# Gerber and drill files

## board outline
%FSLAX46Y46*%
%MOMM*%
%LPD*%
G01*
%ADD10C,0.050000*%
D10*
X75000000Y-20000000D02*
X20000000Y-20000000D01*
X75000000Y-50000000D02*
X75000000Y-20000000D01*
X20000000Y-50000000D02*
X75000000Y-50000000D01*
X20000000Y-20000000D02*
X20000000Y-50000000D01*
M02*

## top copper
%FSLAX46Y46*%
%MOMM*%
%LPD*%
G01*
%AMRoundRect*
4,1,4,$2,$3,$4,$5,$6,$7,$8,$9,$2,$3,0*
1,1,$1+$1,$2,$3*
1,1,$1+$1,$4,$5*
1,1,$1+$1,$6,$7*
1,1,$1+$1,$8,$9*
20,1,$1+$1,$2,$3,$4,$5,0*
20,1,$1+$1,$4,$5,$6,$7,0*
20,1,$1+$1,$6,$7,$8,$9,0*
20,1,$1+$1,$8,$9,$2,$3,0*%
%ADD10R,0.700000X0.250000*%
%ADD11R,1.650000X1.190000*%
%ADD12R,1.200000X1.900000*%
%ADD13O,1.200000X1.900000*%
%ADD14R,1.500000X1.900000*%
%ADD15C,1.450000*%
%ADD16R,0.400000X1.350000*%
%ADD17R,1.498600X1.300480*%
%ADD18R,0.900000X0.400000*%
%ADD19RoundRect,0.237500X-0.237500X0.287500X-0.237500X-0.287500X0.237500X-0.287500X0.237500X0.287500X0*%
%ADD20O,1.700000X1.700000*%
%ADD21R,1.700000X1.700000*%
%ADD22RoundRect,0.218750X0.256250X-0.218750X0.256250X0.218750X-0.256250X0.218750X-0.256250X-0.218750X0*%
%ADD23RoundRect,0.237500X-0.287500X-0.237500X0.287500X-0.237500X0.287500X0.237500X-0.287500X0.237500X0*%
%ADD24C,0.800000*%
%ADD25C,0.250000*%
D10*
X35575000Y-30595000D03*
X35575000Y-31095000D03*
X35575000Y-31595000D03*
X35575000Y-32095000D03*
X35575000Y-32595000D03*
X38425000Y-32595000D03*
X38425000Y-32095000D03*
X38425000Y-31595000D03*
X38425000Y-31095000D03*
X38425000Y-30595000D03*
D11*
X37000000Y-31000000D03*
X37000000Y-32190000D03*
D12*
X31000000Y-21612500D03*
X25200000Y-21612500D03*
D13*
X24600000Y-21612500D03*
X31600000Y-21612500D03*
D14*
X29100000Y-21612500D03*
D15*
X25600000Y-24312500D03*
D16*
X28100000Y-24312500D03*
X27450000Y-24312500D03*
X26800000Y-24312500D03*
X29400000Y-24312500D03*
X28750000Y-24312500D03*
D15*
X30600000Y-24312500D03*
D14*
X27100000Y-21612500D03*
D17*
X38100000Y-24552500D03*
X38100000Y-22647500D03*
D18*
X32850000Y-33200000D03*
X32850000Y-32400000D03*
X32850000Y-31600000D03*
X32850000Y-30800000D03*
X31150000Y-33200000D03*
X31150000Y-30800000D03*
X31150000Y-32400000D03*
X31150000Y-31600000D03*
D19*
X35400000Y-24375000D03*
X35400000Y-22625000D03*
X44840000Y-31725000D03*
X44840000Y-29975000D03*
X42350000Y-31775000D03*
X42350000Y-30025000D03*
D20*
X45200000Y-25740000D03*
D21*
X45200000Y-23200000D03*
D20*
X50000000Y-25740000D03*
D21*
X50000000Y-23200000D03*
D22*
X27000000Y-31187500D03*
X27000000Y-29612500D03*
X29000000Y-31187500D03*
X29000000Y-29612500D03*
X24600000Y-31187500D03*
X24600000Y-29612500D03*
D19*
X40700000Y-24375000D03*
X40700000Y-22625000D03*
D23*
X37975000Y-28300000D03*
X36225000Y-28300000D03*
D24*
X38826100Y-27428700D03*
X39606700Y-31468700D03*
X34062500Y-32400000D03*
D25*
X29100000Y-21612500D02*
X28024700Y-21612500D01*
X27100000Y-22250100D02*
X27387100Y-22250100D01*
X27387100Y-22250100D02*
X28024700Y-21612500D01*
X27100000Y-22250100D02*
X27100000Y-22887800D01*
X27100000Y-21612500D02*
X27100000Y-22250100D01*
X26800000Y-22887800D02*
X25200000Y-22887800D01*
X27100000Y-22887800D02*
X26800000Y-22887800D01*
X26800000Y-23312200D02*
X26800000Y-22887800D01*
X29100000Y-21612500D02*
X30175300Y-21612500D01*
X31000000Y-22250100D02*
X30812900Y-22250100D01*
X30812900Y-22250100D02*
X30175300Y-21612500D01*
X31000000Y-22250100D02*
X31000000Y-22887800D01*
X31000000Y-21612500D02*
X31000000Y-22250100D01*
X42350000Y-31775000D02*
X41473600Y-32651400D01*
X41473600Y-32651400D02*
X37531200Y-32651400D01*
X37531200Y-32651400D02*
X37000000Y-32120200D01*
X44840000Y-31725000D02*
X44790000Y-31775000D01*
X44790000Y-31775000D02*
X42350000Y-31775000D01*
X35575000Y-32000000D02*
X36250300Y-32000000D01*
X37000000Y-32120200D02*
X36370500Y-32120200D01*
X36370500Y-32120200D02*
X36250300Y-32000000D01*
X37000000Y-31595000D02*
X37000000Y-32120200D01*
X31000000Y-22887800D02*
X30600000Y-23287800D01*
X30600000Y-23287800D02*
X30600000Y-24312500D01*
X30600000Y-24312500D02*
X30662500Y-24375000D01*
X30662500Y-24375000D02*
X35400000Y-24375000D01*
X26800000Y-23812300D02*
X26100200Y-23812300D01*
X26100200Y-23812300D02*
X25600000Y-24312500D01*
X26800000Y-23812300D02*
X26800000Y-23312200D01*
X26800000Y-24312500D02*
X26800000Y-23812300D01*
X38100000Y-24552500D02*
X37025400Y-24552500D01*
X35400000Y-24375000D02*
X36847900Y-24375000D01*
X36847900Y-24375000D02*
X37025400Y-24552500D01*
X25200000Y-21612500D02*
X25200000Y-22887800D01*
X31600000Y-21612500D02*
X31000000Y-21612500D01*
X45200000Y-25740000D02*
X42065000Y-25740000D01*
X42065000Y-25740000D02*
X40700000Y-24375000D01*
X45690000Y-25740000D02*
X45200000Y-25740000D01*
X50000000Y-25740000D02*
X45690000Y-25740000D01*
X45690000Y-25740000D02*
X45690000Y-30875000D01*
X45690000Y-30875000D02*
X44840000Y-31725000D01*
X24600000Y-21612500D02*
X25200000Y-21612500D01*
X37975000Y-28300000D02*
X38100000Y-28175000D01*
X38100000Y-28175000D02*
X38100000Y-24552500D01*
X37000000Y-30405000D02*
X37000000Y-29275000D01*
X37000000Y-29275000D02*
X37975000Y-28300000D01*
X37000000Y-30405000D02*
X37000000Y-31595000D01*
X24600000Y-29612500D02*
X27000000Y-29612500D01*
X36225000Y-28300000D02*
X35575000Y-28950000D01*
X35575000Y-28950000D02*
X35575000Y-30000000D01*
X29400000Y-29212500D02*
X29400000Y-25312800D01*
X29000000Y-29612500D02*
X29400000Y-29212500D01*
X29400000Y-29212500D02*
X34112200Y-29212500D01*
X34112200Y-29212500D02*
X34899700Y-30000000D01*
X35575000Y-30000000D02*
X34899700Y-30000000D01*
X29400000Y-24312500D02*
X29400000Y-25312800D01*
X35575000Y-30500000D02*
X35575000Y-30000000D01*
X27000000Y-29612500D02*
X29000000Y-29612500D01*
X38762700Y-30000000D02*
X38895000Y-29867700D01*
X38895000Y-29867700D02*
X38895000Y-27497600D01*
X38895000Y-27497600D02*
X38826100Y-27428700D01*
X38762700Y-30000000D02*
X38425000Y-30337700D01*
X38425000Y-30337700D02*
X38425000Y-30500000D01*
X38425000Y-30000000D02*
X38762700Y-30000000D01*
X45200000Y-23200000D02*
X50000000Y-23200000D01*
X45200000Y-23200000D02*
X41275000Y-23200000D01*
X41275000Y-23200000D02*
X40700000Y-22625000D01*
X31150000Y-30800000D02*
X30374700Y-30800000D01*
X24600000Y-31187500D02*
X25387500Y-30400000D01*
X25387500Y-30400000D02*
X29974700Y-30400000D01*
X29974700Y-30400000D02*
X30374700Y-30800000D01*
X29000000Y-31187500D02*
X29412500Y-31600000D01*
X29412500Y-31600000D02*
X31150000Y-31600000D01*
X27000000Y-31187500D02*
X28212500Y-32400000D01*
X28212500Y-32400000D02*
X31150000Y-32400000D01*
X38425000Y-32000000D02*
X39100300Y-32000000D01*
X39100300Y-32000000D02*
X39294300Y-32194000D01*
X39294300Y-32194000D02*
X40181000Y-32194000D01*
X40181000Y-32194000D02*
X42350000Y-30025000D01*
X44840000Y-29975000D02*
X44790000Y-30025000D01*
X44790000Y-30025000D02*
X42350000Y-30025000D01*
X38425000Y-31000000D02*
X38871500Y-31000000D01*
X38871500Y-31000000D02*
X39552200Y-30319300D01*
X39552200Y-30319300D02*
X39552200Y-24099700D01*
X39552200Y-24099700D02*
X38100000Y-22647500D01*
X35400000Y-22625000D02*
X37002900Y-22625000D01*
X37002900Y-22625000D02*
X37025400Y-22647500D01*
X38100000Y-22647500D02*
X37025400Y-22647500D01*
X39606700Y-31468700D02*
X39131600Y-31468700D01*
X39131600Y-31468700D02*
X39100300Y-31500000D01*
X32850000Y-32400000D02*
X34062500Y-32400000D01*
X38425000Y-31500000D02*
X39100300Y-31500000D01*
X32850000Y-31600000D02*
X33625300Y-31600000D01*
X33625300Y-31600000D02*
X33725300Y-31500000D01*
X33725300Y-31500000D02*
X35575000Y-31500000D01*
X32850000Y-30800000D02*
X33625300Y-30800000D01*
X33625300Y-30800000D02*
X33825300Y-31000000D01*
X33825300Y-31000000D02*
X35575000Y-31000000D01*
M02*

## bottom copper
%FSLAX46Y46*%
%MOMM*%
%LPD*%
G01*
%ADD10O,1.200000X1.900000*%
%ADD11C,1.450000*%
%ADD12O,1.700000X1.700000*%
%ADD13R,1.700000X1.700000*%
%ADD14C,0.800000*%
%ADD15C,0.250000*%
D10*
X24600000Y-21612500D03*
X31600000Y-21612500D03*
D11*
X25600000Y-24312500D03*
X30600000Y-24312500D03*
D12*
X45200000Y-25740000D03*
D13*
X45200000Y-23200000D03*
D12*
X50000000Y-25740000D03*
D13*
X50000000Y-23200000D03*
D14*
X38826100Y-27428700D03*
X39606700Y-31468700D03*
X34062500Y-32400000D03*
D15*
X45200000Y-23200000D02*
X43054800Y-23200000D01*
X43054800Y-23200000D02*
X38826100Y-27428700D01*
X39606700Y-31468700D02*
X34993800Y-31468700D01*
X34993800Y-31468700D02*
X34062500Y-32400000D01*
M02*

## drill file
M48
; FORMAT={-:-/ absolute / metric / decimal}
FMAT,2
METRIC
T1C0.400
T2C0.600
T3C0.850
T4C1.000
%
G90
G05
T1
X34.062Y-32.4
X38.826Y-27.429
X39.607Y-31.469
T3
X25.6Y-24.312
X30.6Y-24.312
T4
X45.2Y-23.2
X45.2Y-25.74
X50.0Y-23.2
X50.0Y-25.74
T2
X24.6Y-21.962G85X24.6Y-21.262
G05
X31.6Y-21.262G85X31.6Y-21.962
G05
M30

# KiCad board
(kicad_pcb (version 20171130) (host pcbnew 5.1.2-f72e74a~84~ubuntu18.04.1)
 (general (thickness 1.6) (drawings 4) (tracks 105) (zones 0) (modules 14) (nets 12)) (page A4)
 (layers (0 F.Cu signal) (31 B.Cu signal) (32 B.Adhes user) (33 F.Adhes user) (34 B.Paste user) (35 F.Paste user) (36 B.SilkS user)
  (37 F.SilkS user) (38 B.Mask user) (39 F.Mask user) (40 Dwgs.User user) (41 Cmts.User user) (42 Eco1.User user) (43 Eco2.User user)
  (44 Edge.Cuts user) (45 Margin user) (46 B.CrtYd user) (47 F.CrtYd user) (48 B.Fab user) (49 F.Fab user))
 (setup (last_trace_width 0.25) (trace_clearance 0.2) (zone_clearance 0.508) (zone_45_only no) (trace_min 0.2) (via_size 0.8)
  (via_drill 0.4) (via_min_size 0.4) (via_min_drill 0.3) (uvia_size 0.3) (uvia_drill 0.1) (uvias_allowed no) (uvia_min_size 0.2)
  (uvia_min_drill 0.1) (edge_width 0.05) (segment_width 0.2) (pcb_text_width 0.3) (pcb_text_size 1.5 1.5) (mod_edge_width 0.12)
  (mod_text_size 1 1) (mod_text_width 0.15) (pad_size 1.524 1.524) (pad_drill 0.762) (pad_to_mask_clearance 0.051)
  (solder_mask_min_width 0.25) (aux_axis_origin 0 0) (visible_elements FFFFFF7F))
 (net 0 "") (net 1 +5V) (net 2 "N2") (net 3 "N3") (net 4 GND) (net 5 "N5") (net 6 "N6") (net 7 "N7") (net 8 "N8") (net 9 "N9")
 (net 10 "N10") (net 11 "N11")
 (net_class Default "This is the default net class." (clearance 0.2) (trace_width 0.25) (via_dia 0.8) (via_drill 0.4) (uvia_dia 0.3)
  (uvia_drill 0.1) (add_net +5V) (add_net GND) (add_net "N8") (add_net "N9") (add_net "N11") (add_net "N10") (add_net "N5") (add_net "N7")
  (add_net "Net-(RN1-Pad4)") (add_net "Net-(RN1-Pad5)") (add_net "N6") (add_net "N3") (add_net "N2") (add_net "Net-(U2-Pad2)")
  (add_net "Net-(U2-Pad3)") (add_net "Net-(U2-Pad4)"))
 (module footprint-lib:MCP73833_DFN (layer F.Cu) (at 37 31.595)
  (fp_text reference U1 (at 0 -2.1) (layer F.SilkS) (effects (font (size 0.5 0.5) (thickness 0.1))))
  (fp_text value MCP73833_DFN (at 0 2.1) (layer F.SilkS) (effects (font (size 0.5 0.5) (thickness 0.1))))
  (pad 1 smd rect (at -1.425 -1) (size 0.7 0.25) (layers F.Cu F.Paste F.Mask) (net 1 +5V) (solder_mask_margin 0.07))
  (pad 2 smd rect (at -1.425 -0.5) (size 0.7 0.25) (layers F.Cu F.Paste F.Mask) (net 1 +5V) (solder_mask_margin 0.07))
  (pad 3 smd rect (at -1.425 0) (size 0.7 0.25) (layers F.Cu F.Paste F.Mask) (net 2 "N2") (solder_mask_margin 0.07))
  (pad 4 smd rect (at -1.425 0.5) (size 0.7 0.25) (layers F.Cu F.Paste F.Mask) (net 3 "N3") (solder_mask_margin 0.07))
  (pad 5 smd rect (at -1.425 1) (size 0.7 0.25) (layers F.Cu F.Paste F.Mask) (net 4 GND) (solder_mask_margin 0.07))
  (pad 6 smd rect (at 1.425 1) (size 0.7 0.25) (layers F.Cu F.Paste F.Mask) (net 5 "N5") (solder_mask_margin 0.07))
  (pad 7 smd rect (at 1.425 0.5) (size 0.7 0.25) (layers F.Cu F.Paste F.Mask) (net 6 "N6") (solder_mask_margin 0.07))
  (pad 8 smd rect (at 1.425 0) (size 0.7 0.25) (layers F.Cu F.Paste F.Mask) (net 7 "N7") (solder_mask_margin 0.07))
  (pad 9 smd rect (at 1.425 -0.5) (size 0.7 0.25) (layers F.Cu F.Paste F.Mask) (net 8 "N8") (solder_mask_margin 0.07))
  (pad 10 smd rect (at 1.425 -1) (size 0.7 0.25) (layers F.Cu F.Paste F.Mask) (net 8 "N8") (solder_mask_margin 0.07))
  (pad 11 smd rect (at 0 -0.595) (size 1.65 1.19) (layers F.Cu F.Paste F.Mask) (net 4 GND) (solder_mask_margin 0.07)
   (solder_paste_margin -0.1))
  (pad 11 smd rect (at 0 0.595) (size 1.65 1.19) (layers F.Cu F.Paste F.Mask) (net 4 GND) (solder_mask_margin 0.07)
   (solder_paste_margin -0.1)))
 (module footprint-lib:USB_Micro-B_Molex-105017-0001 (layer F.Cu) (at 28.1 22.85 180)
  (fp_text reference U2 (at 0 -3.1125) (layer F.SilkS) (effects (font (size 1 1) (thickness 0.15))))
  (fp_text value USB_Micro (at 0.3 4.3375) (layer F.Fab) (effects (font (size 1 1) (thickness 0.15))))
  (pad 6 smd rect (at -2.9 1.2375 180) (size 1.2 1.9) (layers F.Cu F.Mask) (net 4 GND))
  (pad 7 smd rect (at 2.9 1.2375 180) (size 1.2 1.9) (layers F.Cu F.Mask) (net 4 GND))
  (pad 7 thru_hole oval (at 3.5 1.2375 180) (size 1.2 1.9) (drill oval 0.6 1.3) (layers *.Cu *.Mask) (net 4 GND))
  (pad 6 thru_hole oval (at -3.5 1.2375) (size 1.2 1.9) (drill oval 0.6 1.3) (layers *.Cu *.Mask) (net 4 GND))
  (pad 6 smd rect (at -1 1.2375 180) (size 1.5 1.9) (layers F.Cu F.Paste F.Mask) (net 4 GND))
  (pad 9 thru_hole circle (at 2.5 -1.4625 180) (size 1.45 1.45) (drill 0.85) (layers *.Cu *.Mask) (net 4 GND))
  (pad 3 smd rect (at 0 -1.4625 180) (size 0.4 1.35) (layers F.Cu F.Paste F.Mask))
  (pad 4 smd rect (at 0.65 -1.4625 180) (size 0.4 1.35) (layers F.Cu F.Paste F.Mask))
  (pad 5 smd rect (at 1.3 -1.4625 180) (size 0.4 1.35) (layers F.Cu F.Paste F.Mask) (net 4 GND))
  (pad 1 smd rect (at -1.3 -1.4625 180) (size 0.4 1.35) (layers F.Cu F.Paste F.Mask) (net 1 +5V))
  (pad 2 smd rect (at -0.65 -1.4625 180) (size 0.4 1.35) (layers F.Cu F.Paste F.Mask))
  (pad 8 thru_hole circle (at -2.5 -1.4625 180) (size 1.45 1.45) (drill 0.85) (layers *.Cu *.Mask) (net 4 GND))
  (pad 7 smd rect (at 1 1.2375 180) (size 1.5 1.9) (layers F.Cu F.Paste F.Mask) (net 4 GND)))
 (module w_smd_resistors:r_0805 (layer F.Cu) (at 38.1 23.6 90)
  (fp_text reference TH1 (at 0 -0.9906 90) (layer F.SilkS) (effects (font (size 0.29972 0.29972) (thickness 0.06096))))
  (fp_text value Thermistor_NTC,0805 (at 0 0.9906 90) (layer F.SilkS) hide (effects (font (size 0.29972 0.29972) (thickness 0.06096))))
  (pad 2 smd rect (at -0.9525 0 90) (size 1.30048 1.4986) (layers F.Cu F.Paste F.Mask) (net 4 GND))
  (pad 1 smd rect (at 0.9525 0 90) (size 1.30048 1.4986) (layers F.Cu F.Paste F.Mask) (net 7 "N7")))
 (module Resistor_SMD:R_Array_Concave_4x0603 (layer F.Cu) (at 32 32)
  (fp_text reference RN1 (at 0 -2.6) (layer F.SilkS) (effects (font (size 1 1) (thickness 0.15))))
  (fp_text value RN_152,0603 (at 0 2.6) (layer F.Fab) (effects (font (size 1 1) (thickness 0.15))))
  (pad 5 smd rect (at 0.85 1.2) (size 0.9 0.4) (layers F.Cu F.Paste F.Mask))
  (pad 6 smd rect (at 0.85 0.4) (size 0.9 0.4) (layers F.Cu F.Paste F.Mask) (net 6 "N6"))
  (pad 7 smd rect (at 0.85 -0.4) (size 0.9 0.4) (layers F.Cu F.Paste F.Mask) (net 3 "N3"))
  (pad 8 smd rect (at 0.85 -1.2) (size 0.9 0.4) (layers F.Cu F.Paste F.Mask) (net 2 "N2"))
  (pad 4 smd rect (at -0.85 1.2) (size 0.9 0.4) (layers F.Cu F.Paste F.Mask))
  (pad 1 smd rect (at -0.85 -1.2) (size 0.9 0.4) (layers F.Cu F.Paste F.Mask) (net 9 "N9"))
  (pad 3 smd rect (at -0.85 0.4) (size 0.9 0.4) (layers F.Cu F.Paste F.Mask) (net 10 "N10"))
  (pad 2 smd rect (at -0.85 -0.4) (size 0.9 0.4) (layers F.Cu F.Paste F.Mask) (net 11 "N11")))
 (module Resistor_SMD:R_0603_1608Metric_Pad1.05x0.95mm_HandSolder (layer F.Cu) (at 35.4 23.5 270)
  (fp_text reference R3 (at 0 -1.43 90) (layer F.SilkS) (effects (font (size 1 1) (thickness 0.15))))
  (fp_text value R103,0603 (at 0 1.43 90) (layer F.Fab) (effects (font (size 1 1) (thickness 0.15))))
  (pad 2 smd roundrect (at 0.875 0 270) (size 1.05 0.95) (layers F.Cu F.Paste F.Mask) (roundrect_rratio 0.25) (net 4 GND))
  (pad 1 smd roundrect (at -0.875 0 270) (size 1.05 0.95) (layers F.Cu F.Paste F.Mask) (roundrect_rratio 0.25) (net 7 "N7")))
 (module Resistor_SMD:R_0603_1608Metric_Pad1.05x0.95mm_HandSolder (layer F.Cu) (at 44.84 30.85 270)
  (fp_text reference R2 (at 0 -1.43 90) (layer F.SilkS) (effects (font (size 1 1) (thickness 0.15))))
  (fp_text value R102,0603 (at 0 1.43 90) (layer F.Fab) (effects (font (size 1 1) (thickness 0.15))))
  (pad 2 smd roundrect (at 0.875 0 270) (size 1.05 0.95) (layers F.Cu F.Paste F.Mask) (roundrect_rratio 0.25) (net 4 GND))
  (pad 1 smd roundrect (at -0.875 0 270) (size 1.05 0.95) (layers F.Cu F.Paste F.Mask) (roundrect_rratio 0.25) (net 5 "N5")))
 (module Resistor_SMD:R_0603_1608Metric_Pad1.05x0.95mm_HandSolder (layer F.Cu) (at 42.35 30.9 270)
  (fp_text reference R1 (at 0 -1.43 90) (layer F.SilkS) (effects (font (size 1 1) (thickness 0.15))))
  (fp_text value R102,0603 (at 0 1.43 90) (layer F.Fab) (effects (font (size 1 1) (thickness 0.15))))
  (pad 2 smd roundrect (at 0.875 0 270) (size 1.05 0.95) (layers F.Cu F.Paste F.Mask) (roundrect_rratio 0.25) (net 4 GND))
  (pad 1 smd roundrect (at -0.875 0 270) (size 1.05 0.95) (layers F.Cu F.Paste F.Mask) (roundrect_rratio 0.25) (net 5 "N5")))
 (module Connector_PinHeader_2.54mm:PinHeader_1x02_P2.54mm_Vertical (layer F.Cu) (at 45.2 23.2)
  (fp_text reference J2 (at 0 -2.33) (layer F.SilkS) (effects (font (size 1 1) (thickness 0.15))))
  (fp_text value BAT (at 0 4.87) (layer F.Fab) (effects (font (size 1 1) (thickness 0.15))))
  (pad 2 thru_hole oval (at 0 2.54) (size 1.7 1.7) (drill 1) (layers *.Cu *.Mask) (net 4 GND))
  (pad 1 thru_hole rect (at 0 0) (size 1.7 1.7) (drill 1) (layers *.Cu *.Mask) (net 8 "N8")))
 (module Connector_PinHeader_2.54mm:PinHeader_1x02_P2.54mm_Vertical (layer F.Cu) (at 50 23.2)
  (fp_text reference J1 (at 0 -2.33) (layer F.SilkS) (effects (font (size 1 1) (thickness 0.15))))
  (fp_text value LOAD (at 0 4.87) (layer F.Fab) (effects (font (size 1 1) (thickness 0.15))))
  (pad 2 thru_hole oval (at 0 2.54) (size 1.7 1.7) (drill 1) (layers *.Cu *.Mask) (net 4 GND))
  (pad 1 thru_hole rect (at 0 0) (size 1.7 1.7) (drill 1) (layers *.Cu *.Mask) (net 8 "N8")))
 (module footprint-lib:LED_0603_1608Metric (layer F.Cu) (at 27 30.4 90)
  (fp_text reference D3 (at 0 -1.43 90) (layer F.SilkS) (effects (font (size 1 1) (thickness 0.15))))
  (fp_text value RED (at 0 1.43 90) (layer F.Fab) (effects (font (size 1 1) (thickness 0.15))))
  (pad 1 smd roundrect (at -0.7875 0 90) (size 0.875 0.95) (layers F.Cu F.Paste F.Mask) (roundrect_rratio 0.25) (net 10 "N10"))
  (pad 2 smd roundrect (at 0.7875 0 90) (size 0.875 0.95) (layers F.Cu F.Paste F.Mask) (roundrect_rratio 0.25) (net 1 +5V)))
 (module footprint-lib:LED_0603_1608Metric (layer F.Cu) (at 29 30.4 90)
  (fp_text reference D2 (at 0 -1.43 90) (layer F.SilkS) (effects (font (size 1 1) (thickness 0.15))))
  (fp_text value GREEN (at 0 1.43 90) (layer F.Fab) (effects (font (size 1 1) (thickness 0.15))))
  (pad 1 smd roundrect (at -0.7875 0 90) (size 0.875 0.95) (layers F.Cu F.Paste F.Mask) (roundrect_rratio 0.25) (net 11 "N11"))
  (pad 2 smd roundrect (at 0.7875 0 90) (size 0.875 0.95) (layers F.Cu F.Paste F.Mask) (roundrect_rratio 0.25) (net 1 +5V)))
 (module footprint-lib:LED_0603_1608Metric (layer F.Cu) (at 24.6 30.4 90)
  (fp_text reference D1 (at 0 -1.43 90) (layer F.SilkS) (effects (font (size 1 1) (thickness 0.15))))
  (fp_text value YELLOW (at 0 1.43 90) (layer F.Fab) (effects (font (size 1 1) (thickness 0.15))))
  (pad 1 smd roundrect (at -0.7875 0 90) (size 0.875 0.95) (layers F.Cu F.Paste F.Mask) (roundrect_rratio 0.25) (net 9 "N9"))
  (pad 2 smd roundrect (at 0.7875 0 90) (size 0.875 0.95) (layers F.Cu F.Paste F.Mask) (roundrect_rratio 0.25) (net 1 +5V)))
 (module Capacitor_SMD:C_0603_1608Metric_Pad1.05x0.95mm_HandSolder (layer F.Cu) (at 40.7 23.5 270)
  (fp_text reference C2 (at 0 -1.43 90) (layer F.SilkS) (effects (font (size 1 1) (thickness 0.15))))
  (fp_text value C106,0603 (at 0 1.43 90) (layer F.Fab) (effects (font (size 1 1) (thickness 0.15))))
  (pad 2 smd roundrect (at 0.875 0 270) (size 1.05 0.95) (layers F.Cu F.Paste F.Mask) (roundrect_rratio 0.25) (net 4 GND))
  (pad 1 smd roundrect (at -0.875 0 270) (size 1.05 0.95) (layers F.Cu F.Paste F.Mask) (roundrect_rratio 0.25) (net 8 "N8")))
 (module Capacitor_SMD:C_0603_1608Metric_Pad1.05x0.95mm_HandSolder (layer F.Cu) (at 37.1 28.3)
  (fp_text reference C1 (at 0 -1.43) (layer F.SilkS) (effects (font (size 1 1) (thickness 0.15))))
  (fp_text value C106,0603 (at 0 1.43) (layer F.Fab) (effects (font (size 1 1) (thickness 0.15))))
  (pad 2 smd roundrect (at 0.875 0) (size 1.05 0.95) (layers F.Cu F.Paste F.Mask) (roundrect_rratio 0.25) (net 4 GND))
  (pad 1 smd roundrect (at -0.875 0) (size 1.05 0.95) (layers F.Cu F.Paste F.Mask) (roundrect_rratio 0.25) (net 1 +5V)))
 (gr_line (start 75 20) (end 20 20) (layer Edge.Cuts) (width 0.05))
 (gr_line (start 75 50) (end 75 20) (layer Edge.Cuts) (width 0.05))
 (gr_line (start 20 50) (end 75 50) (layer Edge.Cuts) (width 0.05))
 (gr_line (start 20 20) (end 20 50) (layer Edge.Cuts) (width 0.05))
 (segment (start 29.1 21.6125) (end 28.0247 21.6125) (width 0.25) (layer F.Cu) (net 4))
 (segment (start 27.1 22.2501) (end 27.3871 22.2501) (width 0.25) (layer F.Cu) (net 4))
 (segment (start 27.3871 22.2501) (end 28.0247 21.6125) (width 0.25) (layer F.Cu) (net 4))
 (segment (start 27.1 22.2501) (end 27.1 22.8878) (width 0.25) (layer F.Cu) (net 4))
 (segment (start 27.1 21.6125) (end 27.1 22.2501) (width 0.25) (layer F.Cu) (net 4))
 (segment (start 26.8 22.8878) (end 25.2 22.8878) (width 0.25) (layer F.Cu) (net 4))
 (segment (start 27.1 22.8878) (end 26.8 22.8878) (width 0.25) (layer F.Cu) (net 4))
 (segment (start 26.8 23.3122) (end 26.8 22.8878) (width 0.25) (layer F.Cu) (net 4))
 (segment (start 29.1 21.6125) (end 30.1753 21.6125) (width 0.25) (layer F.Cu) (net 4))
 (segment (start 31 22.2501) (end 30.8129 22.2501) (width 0.25) (layer F.Cu) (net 4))
 (segment (start 30.8129 22.2501) (end 30.1753 21.6125) (width 0.25) (layer F.Cu) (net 4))
 (segment (start 31 22.2501) (end 31 22.8878) (width 0.25) (layer F.Cu) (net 4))
 (segment (start 31 21.6125) (end 31 22.2501) (width 0.25) (layer F.Cu) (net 4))
 (segment (start 42.35 31.775) (end 41.4736 32.6514) (width 0.25) (layer F.Cu) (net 4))
 (segment (start 41.4736 32.6514) (end 37.5312 32.6514) (width 0.25) (layer F.Cu) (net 4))
 (segment (start 37.5312 32.6514) (end 37 32.1202) (width 0.25) (layer F.Cu) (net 4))
 (segment (start 44.84 31.725) (end 44.79 31.775) (width 0.25) (layer F.Cu) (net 4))
 (segment (start 44.79 31.775) (end 42.35 31.775) (width 0.25) (layer F.Cu) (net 4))
 (segment (start 35.575 32) (end 36.2503 32) (width 0.25) (layer F.Cu) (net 4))
 (segment (start 37 32.1202) (end 36.3705 32.1202) (width 0.25) (layer F.Cu) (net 4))
 (segment (start 36.3705 32.1202) (end 36.2503 32) (width 0.25) (layer F.Cu) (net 4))
 (segment (start 37 31.595) (end 37 32.1202) (width 0.25) (layer F.Cu) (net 4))
 (segment (start 31 22.8878) (end 30.6 23.2878) (width 0.25) (layer F.Cu) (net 4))
 (segment (start 30.6 23.2878) (end 30.6 24.3125) (width 0.25) (layer F.Cu) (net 4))
 (segment (start 30.6 24.3125) (end 30.6625 24.375) (width 0.25) (layer F.Cu) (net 4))
 (segment (start 30.6625 24.375) (end 35.4 24.375) (width 0.25) (layer F.Cu) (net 4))
 (segment (start 26.8 23.8123) (end 26.1002 23.8123) (width 0.25) (layer F.Cu) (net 4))
 (segment (start 26.1002 23.8123) (end 25.6 24.3125) (width 0.25) (layer F.Cu) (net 4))
 (segment (start 26.8 23.8123) (end 26.8 23.3122) (width 0.25) (layer F.Cu) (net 4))
 (segment (start 26.8 24.3125) (end 26.8 23.8123) (width 0.25) (layer F.Cu) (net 4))
 (segment (start 38.1 24.5525) (end 37.0254 24.5525) (width 0.25) (layer F.Cu) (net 4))
 (segment (start 35.4 24.375) (end 36.8479 24.375) (width 0.25) (layer F.Cu) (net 4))
 (segment (start 36.8479 24.375) (end 37.0254 24.5525) (width 0.25) (layer F.Cu) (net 4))
 (segment (start 25.2 21.6125) (end 25.2 22.8878) (width 0.25) (layer F.Cu) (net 4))
 (segment (start 31.6 21.6125) (end 31 21.6125) (width 0.25) (layer F.Cu) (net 4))
 (segment (start 45.2 25.74) (end 42.065 25.74) (width 0.25) (layer F.Cu) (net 4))
 (segment (start 42.065 25.74) (end 40.7 24.375) (width 0.25) (layer F.Cu) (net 4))
 (segment (start 45.69 25.74) (end 45.2 25.74) (width 0.25) (layer F.Cu) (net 4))
 (segment (start 50 25.74) (end 45.69 25.74) (width 0.25) (layer F.Cu) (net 4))
 (segment (start 45.69 25.74) (end 45.69 30.875) (width 0.25) (layer F.Cu) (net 4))
 (segment (start 45.69 30.875) (end 44.84 31.725) (width 0.25) (layer F.Cu) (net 4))
 (segment (start 24.6 21.6125) (end 25.2 21.6125) (width 0.25) (layer F.Cu) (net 4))
 (segment (start 37.975 28.3) (end 38.1 28.175) (width 0.25) (layer F.Cu) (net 4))
 (segment (start 38.1 28.175) (end 38.1 24.5525) (width 0.25) (layer F.Cu) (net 4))
 (segment (start 37 30.405) (end 37 29.275) (width 0.25) (layer F.Cu) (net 4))
 (segment (start 37 29.275) (end 37.975 28.3) (width 0.25) (layer F.Cu) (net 4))
 (segment (start 37 30.405) (end 37 31.595) (width 0.25) (layer F.Cu) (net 4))
 (segment (start 24.6 29.6125) (end 27 29.6125) (width 0.25) (layer F.Cu) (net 1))
 (segment (start 36.225 28.3) (end 35.575 28.95) (width 0.25) (layer F.Cu) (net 1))
 (segment (start 35.575 28.95) (end 35.575 30) (width 0.25) (layer F.Cu) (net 1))
 (segment (start 29.4 29.2125) (end 29.4 25.3128) (width 0.25) (layer F.Cu) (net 1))
 (segment (start 29 29.6125) (end 29.4 29.2125) (width 0.25) (layer F.Cu) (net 1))
 (segment (start 29.4 29.2125) (end 34.1122 29.2125) (width 0.25) (layer F.Cu) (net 1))
 (segment (start 34.1122 29.2125) (end 34.8997 30) (width 0.25) (layer F.Cu) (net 1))
 (segment (start 35.575 30) (end 34.8997 30) (width 0.25) (layer F.Cu) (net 1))
 (segment (start 29.4 24.3125) (end 29.4 25.3128) (width 0.25) (layer F.Cu) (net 1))
 (segment (start 35.575 30.5) (end 35.575 30) (width 0.25) (layer F.Cu) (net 1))
 (segment (start 27 29.6125) (end 29 29.6125) (width 0.25) (layer F.Cu) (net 1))
 (segment (start 38.7627 30) (end 38.895 29.8677) (width 0.25) (layer F.Cu) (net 8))
 (segment (start 38.895 29.8677) (end 38.895 27.4976) (width 0.25) (layer F.Cu) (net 8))
 (segment (start 38.895 27.4976) (end 38.8261 27.4287) (width 0.25) (layer F.Cu) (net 8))
 (segment (start 45.2 23.2) (end 43.0548 23.2) (width 0.25) (layer B.Cu) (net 8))
 (segment (start 43.0548 23.2) (end 38.8261 27.4287) (width 0.25) (layer B.Cu) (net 8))
 (segment (start 38.7627 30) (end 38.425 30.3377) (width 0.25) (layer F.Cu) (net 8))
 (segment (start 38.425 30.3377) (end 38.425 30.5) (width 0.25) (layer F.Cu) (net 8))
 (segment (start 38.425 30) (end 38.7627 30) (width 0.25) (layer F.Cu) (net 8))
 (segment (start 45.2 23.2) (end 50 23.2) (width 0.25) (layer F.Cu) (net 8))
 (segment (start 45.2 23.2) (end 41.275 23.2) (width 0.25) (layer F.Cu) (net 8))
 (segment (start 41.275 23.2) (end 40.7 22.625) (width 0.25) (layer F.Cu) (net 8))
 (via (at 38.8261 27.4287) (size 0.8) (layers F.Cu B.Cu) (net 8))
 (segment (start 31.15 30.8) (end 30.3747 30.8) (width 0.25) (layer F.Cu) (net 9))
 (segment (start 24.6 31.1875) (end 25.3875 30.4) (width 0.25) (layer F.Cu) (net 9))
 (segment (start 25.3875 30.4) (end 29.9747 30.4) (width 0.25) (layer F.Cu) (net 9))
 (segment (start 29.9747 30.4) (end 30.3747 30.8) (width 0.25) (layer F.Cu) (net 9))
 (segment (start 29 31.1875) (end 29.4125 31.6) (width 0.25) (layer F.Cu) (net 11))
 (segment (start 29.4125 31.6) (end 31.15 31.6) (width 0.25) (layer F.Cu) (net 11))
 (segment (start 27 31.1875) (end 28.2125 32.4) (width 0.25) (layer F.Cu) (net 10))
 (segment (start 28.2125 32.4) (end 31.15 32.4) (width 0.25) (layer F.Cu) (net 10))
 (segment (start 38.425 32) (end 39.1003 32) (width 0.25) (layer F.Cu) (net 5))
 (segment (start 39.1003 32) (end 39.2943 32.194) (width 0.25) (layer F.Cu) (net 5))
 (segment (start 39.2943 32.194) (end 40.181 32.194) (width 0.25) (layer F.Cu) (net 5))
 (segment (start 40.181 32.194) (end 42.35 30.025) (width 0.25) (layer F.Cu) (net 5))
 (segment (start 44.84 29.975) (end 44.79 30.025) (width 0.25) (layer F.Cu) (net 5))
 (segment (start 44.79 30.025) (end 42.35 30.025) (width 0.25) (layer F.Cu) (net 5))
 (segment (start 38.425 31) (end 38.8715 31) (width 0.25) (layer F.Cu) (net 7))
 (segment (start 38.8715 31) (end 39.5522 30.3193) (width 0.25) (layer F.Cu) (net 7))
 (segment (start 39.5522 30.3193) (end 39.5522 24.0997) (width 0.25) (layer F.Cu) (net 7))
 (segment (start 39.5522 24.0997) (end 38.1 22.6475) (width 0.25) (layer F.Cu) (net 7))
 (segment (start 35.4 22.625) (end 37.0029 22.625) (width 0.25) (layer F.Cu) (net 7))
 (segment (start 37.0029 22.625) (end 37.0254 22.6475) (width 0.25) (layer F.Cu) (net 7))
 (segment (start 38.1 22.6475) (end 37.0254 22.6475) (width 0.25) (layer F.Cu) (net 7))
 (segment (start 39.6067 31.4687) (end 39.1316 31.4687) (width 0.25) (layer F.Cu) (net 6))
 (segment (start 39.1316 31.4687) (end 39.1003 31.5) (width 0.25) (layer F.Cu) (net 6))
 (segment (start 39.6067 31.4687) (end 34.9938 31.4687) (width 0.25) (layer B.Cu) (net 6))
 (segment (start 34.9938 31.4687) (end 34.0625 32.4) (width 0.25) (layer B.Cu) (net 6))
 (segment (start 32.85 32.4) (end 34.0625 32.4) (width 0.25) (layer F.Cu) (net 6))
 (segment (start 38.425 31.5) (end 39.1003 31.5) (width 0.25) (layer F.Cu) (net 6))
 (via (at 39.6067 31.4687) (size 0.8) (layers F.Cu B.Cu) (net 6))
 (via (at 34.0625 32.4) (size 0.8) (layers F.Cu B.Cu) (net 6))
 (segment (start 32.85 31.6) (end 33.6253 31.6) (width 0.25) (layer F.Cu) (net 3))
 (segment (start 33.6253 31.6) (end 33.7253 31.5) (width 0.25) (layer F.Cu) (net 3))
 (segment (start 33.7253 31.5) (end 35.575 31.5) (width 0.25) (layer F.Cu) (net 3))
 (segment (start 32.85 30.8) (end 33.6253 30.8) (width 0.25) (layer F.Cu) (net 2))
 (segment (start 33.6253 30.8) (end 33.8253 31) (width 0.25) (layer F.Cu) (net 2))
 (segment (start 33.8253 31) (end 35.575 31) (width 0.25) (layer F.Cu) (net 2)))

